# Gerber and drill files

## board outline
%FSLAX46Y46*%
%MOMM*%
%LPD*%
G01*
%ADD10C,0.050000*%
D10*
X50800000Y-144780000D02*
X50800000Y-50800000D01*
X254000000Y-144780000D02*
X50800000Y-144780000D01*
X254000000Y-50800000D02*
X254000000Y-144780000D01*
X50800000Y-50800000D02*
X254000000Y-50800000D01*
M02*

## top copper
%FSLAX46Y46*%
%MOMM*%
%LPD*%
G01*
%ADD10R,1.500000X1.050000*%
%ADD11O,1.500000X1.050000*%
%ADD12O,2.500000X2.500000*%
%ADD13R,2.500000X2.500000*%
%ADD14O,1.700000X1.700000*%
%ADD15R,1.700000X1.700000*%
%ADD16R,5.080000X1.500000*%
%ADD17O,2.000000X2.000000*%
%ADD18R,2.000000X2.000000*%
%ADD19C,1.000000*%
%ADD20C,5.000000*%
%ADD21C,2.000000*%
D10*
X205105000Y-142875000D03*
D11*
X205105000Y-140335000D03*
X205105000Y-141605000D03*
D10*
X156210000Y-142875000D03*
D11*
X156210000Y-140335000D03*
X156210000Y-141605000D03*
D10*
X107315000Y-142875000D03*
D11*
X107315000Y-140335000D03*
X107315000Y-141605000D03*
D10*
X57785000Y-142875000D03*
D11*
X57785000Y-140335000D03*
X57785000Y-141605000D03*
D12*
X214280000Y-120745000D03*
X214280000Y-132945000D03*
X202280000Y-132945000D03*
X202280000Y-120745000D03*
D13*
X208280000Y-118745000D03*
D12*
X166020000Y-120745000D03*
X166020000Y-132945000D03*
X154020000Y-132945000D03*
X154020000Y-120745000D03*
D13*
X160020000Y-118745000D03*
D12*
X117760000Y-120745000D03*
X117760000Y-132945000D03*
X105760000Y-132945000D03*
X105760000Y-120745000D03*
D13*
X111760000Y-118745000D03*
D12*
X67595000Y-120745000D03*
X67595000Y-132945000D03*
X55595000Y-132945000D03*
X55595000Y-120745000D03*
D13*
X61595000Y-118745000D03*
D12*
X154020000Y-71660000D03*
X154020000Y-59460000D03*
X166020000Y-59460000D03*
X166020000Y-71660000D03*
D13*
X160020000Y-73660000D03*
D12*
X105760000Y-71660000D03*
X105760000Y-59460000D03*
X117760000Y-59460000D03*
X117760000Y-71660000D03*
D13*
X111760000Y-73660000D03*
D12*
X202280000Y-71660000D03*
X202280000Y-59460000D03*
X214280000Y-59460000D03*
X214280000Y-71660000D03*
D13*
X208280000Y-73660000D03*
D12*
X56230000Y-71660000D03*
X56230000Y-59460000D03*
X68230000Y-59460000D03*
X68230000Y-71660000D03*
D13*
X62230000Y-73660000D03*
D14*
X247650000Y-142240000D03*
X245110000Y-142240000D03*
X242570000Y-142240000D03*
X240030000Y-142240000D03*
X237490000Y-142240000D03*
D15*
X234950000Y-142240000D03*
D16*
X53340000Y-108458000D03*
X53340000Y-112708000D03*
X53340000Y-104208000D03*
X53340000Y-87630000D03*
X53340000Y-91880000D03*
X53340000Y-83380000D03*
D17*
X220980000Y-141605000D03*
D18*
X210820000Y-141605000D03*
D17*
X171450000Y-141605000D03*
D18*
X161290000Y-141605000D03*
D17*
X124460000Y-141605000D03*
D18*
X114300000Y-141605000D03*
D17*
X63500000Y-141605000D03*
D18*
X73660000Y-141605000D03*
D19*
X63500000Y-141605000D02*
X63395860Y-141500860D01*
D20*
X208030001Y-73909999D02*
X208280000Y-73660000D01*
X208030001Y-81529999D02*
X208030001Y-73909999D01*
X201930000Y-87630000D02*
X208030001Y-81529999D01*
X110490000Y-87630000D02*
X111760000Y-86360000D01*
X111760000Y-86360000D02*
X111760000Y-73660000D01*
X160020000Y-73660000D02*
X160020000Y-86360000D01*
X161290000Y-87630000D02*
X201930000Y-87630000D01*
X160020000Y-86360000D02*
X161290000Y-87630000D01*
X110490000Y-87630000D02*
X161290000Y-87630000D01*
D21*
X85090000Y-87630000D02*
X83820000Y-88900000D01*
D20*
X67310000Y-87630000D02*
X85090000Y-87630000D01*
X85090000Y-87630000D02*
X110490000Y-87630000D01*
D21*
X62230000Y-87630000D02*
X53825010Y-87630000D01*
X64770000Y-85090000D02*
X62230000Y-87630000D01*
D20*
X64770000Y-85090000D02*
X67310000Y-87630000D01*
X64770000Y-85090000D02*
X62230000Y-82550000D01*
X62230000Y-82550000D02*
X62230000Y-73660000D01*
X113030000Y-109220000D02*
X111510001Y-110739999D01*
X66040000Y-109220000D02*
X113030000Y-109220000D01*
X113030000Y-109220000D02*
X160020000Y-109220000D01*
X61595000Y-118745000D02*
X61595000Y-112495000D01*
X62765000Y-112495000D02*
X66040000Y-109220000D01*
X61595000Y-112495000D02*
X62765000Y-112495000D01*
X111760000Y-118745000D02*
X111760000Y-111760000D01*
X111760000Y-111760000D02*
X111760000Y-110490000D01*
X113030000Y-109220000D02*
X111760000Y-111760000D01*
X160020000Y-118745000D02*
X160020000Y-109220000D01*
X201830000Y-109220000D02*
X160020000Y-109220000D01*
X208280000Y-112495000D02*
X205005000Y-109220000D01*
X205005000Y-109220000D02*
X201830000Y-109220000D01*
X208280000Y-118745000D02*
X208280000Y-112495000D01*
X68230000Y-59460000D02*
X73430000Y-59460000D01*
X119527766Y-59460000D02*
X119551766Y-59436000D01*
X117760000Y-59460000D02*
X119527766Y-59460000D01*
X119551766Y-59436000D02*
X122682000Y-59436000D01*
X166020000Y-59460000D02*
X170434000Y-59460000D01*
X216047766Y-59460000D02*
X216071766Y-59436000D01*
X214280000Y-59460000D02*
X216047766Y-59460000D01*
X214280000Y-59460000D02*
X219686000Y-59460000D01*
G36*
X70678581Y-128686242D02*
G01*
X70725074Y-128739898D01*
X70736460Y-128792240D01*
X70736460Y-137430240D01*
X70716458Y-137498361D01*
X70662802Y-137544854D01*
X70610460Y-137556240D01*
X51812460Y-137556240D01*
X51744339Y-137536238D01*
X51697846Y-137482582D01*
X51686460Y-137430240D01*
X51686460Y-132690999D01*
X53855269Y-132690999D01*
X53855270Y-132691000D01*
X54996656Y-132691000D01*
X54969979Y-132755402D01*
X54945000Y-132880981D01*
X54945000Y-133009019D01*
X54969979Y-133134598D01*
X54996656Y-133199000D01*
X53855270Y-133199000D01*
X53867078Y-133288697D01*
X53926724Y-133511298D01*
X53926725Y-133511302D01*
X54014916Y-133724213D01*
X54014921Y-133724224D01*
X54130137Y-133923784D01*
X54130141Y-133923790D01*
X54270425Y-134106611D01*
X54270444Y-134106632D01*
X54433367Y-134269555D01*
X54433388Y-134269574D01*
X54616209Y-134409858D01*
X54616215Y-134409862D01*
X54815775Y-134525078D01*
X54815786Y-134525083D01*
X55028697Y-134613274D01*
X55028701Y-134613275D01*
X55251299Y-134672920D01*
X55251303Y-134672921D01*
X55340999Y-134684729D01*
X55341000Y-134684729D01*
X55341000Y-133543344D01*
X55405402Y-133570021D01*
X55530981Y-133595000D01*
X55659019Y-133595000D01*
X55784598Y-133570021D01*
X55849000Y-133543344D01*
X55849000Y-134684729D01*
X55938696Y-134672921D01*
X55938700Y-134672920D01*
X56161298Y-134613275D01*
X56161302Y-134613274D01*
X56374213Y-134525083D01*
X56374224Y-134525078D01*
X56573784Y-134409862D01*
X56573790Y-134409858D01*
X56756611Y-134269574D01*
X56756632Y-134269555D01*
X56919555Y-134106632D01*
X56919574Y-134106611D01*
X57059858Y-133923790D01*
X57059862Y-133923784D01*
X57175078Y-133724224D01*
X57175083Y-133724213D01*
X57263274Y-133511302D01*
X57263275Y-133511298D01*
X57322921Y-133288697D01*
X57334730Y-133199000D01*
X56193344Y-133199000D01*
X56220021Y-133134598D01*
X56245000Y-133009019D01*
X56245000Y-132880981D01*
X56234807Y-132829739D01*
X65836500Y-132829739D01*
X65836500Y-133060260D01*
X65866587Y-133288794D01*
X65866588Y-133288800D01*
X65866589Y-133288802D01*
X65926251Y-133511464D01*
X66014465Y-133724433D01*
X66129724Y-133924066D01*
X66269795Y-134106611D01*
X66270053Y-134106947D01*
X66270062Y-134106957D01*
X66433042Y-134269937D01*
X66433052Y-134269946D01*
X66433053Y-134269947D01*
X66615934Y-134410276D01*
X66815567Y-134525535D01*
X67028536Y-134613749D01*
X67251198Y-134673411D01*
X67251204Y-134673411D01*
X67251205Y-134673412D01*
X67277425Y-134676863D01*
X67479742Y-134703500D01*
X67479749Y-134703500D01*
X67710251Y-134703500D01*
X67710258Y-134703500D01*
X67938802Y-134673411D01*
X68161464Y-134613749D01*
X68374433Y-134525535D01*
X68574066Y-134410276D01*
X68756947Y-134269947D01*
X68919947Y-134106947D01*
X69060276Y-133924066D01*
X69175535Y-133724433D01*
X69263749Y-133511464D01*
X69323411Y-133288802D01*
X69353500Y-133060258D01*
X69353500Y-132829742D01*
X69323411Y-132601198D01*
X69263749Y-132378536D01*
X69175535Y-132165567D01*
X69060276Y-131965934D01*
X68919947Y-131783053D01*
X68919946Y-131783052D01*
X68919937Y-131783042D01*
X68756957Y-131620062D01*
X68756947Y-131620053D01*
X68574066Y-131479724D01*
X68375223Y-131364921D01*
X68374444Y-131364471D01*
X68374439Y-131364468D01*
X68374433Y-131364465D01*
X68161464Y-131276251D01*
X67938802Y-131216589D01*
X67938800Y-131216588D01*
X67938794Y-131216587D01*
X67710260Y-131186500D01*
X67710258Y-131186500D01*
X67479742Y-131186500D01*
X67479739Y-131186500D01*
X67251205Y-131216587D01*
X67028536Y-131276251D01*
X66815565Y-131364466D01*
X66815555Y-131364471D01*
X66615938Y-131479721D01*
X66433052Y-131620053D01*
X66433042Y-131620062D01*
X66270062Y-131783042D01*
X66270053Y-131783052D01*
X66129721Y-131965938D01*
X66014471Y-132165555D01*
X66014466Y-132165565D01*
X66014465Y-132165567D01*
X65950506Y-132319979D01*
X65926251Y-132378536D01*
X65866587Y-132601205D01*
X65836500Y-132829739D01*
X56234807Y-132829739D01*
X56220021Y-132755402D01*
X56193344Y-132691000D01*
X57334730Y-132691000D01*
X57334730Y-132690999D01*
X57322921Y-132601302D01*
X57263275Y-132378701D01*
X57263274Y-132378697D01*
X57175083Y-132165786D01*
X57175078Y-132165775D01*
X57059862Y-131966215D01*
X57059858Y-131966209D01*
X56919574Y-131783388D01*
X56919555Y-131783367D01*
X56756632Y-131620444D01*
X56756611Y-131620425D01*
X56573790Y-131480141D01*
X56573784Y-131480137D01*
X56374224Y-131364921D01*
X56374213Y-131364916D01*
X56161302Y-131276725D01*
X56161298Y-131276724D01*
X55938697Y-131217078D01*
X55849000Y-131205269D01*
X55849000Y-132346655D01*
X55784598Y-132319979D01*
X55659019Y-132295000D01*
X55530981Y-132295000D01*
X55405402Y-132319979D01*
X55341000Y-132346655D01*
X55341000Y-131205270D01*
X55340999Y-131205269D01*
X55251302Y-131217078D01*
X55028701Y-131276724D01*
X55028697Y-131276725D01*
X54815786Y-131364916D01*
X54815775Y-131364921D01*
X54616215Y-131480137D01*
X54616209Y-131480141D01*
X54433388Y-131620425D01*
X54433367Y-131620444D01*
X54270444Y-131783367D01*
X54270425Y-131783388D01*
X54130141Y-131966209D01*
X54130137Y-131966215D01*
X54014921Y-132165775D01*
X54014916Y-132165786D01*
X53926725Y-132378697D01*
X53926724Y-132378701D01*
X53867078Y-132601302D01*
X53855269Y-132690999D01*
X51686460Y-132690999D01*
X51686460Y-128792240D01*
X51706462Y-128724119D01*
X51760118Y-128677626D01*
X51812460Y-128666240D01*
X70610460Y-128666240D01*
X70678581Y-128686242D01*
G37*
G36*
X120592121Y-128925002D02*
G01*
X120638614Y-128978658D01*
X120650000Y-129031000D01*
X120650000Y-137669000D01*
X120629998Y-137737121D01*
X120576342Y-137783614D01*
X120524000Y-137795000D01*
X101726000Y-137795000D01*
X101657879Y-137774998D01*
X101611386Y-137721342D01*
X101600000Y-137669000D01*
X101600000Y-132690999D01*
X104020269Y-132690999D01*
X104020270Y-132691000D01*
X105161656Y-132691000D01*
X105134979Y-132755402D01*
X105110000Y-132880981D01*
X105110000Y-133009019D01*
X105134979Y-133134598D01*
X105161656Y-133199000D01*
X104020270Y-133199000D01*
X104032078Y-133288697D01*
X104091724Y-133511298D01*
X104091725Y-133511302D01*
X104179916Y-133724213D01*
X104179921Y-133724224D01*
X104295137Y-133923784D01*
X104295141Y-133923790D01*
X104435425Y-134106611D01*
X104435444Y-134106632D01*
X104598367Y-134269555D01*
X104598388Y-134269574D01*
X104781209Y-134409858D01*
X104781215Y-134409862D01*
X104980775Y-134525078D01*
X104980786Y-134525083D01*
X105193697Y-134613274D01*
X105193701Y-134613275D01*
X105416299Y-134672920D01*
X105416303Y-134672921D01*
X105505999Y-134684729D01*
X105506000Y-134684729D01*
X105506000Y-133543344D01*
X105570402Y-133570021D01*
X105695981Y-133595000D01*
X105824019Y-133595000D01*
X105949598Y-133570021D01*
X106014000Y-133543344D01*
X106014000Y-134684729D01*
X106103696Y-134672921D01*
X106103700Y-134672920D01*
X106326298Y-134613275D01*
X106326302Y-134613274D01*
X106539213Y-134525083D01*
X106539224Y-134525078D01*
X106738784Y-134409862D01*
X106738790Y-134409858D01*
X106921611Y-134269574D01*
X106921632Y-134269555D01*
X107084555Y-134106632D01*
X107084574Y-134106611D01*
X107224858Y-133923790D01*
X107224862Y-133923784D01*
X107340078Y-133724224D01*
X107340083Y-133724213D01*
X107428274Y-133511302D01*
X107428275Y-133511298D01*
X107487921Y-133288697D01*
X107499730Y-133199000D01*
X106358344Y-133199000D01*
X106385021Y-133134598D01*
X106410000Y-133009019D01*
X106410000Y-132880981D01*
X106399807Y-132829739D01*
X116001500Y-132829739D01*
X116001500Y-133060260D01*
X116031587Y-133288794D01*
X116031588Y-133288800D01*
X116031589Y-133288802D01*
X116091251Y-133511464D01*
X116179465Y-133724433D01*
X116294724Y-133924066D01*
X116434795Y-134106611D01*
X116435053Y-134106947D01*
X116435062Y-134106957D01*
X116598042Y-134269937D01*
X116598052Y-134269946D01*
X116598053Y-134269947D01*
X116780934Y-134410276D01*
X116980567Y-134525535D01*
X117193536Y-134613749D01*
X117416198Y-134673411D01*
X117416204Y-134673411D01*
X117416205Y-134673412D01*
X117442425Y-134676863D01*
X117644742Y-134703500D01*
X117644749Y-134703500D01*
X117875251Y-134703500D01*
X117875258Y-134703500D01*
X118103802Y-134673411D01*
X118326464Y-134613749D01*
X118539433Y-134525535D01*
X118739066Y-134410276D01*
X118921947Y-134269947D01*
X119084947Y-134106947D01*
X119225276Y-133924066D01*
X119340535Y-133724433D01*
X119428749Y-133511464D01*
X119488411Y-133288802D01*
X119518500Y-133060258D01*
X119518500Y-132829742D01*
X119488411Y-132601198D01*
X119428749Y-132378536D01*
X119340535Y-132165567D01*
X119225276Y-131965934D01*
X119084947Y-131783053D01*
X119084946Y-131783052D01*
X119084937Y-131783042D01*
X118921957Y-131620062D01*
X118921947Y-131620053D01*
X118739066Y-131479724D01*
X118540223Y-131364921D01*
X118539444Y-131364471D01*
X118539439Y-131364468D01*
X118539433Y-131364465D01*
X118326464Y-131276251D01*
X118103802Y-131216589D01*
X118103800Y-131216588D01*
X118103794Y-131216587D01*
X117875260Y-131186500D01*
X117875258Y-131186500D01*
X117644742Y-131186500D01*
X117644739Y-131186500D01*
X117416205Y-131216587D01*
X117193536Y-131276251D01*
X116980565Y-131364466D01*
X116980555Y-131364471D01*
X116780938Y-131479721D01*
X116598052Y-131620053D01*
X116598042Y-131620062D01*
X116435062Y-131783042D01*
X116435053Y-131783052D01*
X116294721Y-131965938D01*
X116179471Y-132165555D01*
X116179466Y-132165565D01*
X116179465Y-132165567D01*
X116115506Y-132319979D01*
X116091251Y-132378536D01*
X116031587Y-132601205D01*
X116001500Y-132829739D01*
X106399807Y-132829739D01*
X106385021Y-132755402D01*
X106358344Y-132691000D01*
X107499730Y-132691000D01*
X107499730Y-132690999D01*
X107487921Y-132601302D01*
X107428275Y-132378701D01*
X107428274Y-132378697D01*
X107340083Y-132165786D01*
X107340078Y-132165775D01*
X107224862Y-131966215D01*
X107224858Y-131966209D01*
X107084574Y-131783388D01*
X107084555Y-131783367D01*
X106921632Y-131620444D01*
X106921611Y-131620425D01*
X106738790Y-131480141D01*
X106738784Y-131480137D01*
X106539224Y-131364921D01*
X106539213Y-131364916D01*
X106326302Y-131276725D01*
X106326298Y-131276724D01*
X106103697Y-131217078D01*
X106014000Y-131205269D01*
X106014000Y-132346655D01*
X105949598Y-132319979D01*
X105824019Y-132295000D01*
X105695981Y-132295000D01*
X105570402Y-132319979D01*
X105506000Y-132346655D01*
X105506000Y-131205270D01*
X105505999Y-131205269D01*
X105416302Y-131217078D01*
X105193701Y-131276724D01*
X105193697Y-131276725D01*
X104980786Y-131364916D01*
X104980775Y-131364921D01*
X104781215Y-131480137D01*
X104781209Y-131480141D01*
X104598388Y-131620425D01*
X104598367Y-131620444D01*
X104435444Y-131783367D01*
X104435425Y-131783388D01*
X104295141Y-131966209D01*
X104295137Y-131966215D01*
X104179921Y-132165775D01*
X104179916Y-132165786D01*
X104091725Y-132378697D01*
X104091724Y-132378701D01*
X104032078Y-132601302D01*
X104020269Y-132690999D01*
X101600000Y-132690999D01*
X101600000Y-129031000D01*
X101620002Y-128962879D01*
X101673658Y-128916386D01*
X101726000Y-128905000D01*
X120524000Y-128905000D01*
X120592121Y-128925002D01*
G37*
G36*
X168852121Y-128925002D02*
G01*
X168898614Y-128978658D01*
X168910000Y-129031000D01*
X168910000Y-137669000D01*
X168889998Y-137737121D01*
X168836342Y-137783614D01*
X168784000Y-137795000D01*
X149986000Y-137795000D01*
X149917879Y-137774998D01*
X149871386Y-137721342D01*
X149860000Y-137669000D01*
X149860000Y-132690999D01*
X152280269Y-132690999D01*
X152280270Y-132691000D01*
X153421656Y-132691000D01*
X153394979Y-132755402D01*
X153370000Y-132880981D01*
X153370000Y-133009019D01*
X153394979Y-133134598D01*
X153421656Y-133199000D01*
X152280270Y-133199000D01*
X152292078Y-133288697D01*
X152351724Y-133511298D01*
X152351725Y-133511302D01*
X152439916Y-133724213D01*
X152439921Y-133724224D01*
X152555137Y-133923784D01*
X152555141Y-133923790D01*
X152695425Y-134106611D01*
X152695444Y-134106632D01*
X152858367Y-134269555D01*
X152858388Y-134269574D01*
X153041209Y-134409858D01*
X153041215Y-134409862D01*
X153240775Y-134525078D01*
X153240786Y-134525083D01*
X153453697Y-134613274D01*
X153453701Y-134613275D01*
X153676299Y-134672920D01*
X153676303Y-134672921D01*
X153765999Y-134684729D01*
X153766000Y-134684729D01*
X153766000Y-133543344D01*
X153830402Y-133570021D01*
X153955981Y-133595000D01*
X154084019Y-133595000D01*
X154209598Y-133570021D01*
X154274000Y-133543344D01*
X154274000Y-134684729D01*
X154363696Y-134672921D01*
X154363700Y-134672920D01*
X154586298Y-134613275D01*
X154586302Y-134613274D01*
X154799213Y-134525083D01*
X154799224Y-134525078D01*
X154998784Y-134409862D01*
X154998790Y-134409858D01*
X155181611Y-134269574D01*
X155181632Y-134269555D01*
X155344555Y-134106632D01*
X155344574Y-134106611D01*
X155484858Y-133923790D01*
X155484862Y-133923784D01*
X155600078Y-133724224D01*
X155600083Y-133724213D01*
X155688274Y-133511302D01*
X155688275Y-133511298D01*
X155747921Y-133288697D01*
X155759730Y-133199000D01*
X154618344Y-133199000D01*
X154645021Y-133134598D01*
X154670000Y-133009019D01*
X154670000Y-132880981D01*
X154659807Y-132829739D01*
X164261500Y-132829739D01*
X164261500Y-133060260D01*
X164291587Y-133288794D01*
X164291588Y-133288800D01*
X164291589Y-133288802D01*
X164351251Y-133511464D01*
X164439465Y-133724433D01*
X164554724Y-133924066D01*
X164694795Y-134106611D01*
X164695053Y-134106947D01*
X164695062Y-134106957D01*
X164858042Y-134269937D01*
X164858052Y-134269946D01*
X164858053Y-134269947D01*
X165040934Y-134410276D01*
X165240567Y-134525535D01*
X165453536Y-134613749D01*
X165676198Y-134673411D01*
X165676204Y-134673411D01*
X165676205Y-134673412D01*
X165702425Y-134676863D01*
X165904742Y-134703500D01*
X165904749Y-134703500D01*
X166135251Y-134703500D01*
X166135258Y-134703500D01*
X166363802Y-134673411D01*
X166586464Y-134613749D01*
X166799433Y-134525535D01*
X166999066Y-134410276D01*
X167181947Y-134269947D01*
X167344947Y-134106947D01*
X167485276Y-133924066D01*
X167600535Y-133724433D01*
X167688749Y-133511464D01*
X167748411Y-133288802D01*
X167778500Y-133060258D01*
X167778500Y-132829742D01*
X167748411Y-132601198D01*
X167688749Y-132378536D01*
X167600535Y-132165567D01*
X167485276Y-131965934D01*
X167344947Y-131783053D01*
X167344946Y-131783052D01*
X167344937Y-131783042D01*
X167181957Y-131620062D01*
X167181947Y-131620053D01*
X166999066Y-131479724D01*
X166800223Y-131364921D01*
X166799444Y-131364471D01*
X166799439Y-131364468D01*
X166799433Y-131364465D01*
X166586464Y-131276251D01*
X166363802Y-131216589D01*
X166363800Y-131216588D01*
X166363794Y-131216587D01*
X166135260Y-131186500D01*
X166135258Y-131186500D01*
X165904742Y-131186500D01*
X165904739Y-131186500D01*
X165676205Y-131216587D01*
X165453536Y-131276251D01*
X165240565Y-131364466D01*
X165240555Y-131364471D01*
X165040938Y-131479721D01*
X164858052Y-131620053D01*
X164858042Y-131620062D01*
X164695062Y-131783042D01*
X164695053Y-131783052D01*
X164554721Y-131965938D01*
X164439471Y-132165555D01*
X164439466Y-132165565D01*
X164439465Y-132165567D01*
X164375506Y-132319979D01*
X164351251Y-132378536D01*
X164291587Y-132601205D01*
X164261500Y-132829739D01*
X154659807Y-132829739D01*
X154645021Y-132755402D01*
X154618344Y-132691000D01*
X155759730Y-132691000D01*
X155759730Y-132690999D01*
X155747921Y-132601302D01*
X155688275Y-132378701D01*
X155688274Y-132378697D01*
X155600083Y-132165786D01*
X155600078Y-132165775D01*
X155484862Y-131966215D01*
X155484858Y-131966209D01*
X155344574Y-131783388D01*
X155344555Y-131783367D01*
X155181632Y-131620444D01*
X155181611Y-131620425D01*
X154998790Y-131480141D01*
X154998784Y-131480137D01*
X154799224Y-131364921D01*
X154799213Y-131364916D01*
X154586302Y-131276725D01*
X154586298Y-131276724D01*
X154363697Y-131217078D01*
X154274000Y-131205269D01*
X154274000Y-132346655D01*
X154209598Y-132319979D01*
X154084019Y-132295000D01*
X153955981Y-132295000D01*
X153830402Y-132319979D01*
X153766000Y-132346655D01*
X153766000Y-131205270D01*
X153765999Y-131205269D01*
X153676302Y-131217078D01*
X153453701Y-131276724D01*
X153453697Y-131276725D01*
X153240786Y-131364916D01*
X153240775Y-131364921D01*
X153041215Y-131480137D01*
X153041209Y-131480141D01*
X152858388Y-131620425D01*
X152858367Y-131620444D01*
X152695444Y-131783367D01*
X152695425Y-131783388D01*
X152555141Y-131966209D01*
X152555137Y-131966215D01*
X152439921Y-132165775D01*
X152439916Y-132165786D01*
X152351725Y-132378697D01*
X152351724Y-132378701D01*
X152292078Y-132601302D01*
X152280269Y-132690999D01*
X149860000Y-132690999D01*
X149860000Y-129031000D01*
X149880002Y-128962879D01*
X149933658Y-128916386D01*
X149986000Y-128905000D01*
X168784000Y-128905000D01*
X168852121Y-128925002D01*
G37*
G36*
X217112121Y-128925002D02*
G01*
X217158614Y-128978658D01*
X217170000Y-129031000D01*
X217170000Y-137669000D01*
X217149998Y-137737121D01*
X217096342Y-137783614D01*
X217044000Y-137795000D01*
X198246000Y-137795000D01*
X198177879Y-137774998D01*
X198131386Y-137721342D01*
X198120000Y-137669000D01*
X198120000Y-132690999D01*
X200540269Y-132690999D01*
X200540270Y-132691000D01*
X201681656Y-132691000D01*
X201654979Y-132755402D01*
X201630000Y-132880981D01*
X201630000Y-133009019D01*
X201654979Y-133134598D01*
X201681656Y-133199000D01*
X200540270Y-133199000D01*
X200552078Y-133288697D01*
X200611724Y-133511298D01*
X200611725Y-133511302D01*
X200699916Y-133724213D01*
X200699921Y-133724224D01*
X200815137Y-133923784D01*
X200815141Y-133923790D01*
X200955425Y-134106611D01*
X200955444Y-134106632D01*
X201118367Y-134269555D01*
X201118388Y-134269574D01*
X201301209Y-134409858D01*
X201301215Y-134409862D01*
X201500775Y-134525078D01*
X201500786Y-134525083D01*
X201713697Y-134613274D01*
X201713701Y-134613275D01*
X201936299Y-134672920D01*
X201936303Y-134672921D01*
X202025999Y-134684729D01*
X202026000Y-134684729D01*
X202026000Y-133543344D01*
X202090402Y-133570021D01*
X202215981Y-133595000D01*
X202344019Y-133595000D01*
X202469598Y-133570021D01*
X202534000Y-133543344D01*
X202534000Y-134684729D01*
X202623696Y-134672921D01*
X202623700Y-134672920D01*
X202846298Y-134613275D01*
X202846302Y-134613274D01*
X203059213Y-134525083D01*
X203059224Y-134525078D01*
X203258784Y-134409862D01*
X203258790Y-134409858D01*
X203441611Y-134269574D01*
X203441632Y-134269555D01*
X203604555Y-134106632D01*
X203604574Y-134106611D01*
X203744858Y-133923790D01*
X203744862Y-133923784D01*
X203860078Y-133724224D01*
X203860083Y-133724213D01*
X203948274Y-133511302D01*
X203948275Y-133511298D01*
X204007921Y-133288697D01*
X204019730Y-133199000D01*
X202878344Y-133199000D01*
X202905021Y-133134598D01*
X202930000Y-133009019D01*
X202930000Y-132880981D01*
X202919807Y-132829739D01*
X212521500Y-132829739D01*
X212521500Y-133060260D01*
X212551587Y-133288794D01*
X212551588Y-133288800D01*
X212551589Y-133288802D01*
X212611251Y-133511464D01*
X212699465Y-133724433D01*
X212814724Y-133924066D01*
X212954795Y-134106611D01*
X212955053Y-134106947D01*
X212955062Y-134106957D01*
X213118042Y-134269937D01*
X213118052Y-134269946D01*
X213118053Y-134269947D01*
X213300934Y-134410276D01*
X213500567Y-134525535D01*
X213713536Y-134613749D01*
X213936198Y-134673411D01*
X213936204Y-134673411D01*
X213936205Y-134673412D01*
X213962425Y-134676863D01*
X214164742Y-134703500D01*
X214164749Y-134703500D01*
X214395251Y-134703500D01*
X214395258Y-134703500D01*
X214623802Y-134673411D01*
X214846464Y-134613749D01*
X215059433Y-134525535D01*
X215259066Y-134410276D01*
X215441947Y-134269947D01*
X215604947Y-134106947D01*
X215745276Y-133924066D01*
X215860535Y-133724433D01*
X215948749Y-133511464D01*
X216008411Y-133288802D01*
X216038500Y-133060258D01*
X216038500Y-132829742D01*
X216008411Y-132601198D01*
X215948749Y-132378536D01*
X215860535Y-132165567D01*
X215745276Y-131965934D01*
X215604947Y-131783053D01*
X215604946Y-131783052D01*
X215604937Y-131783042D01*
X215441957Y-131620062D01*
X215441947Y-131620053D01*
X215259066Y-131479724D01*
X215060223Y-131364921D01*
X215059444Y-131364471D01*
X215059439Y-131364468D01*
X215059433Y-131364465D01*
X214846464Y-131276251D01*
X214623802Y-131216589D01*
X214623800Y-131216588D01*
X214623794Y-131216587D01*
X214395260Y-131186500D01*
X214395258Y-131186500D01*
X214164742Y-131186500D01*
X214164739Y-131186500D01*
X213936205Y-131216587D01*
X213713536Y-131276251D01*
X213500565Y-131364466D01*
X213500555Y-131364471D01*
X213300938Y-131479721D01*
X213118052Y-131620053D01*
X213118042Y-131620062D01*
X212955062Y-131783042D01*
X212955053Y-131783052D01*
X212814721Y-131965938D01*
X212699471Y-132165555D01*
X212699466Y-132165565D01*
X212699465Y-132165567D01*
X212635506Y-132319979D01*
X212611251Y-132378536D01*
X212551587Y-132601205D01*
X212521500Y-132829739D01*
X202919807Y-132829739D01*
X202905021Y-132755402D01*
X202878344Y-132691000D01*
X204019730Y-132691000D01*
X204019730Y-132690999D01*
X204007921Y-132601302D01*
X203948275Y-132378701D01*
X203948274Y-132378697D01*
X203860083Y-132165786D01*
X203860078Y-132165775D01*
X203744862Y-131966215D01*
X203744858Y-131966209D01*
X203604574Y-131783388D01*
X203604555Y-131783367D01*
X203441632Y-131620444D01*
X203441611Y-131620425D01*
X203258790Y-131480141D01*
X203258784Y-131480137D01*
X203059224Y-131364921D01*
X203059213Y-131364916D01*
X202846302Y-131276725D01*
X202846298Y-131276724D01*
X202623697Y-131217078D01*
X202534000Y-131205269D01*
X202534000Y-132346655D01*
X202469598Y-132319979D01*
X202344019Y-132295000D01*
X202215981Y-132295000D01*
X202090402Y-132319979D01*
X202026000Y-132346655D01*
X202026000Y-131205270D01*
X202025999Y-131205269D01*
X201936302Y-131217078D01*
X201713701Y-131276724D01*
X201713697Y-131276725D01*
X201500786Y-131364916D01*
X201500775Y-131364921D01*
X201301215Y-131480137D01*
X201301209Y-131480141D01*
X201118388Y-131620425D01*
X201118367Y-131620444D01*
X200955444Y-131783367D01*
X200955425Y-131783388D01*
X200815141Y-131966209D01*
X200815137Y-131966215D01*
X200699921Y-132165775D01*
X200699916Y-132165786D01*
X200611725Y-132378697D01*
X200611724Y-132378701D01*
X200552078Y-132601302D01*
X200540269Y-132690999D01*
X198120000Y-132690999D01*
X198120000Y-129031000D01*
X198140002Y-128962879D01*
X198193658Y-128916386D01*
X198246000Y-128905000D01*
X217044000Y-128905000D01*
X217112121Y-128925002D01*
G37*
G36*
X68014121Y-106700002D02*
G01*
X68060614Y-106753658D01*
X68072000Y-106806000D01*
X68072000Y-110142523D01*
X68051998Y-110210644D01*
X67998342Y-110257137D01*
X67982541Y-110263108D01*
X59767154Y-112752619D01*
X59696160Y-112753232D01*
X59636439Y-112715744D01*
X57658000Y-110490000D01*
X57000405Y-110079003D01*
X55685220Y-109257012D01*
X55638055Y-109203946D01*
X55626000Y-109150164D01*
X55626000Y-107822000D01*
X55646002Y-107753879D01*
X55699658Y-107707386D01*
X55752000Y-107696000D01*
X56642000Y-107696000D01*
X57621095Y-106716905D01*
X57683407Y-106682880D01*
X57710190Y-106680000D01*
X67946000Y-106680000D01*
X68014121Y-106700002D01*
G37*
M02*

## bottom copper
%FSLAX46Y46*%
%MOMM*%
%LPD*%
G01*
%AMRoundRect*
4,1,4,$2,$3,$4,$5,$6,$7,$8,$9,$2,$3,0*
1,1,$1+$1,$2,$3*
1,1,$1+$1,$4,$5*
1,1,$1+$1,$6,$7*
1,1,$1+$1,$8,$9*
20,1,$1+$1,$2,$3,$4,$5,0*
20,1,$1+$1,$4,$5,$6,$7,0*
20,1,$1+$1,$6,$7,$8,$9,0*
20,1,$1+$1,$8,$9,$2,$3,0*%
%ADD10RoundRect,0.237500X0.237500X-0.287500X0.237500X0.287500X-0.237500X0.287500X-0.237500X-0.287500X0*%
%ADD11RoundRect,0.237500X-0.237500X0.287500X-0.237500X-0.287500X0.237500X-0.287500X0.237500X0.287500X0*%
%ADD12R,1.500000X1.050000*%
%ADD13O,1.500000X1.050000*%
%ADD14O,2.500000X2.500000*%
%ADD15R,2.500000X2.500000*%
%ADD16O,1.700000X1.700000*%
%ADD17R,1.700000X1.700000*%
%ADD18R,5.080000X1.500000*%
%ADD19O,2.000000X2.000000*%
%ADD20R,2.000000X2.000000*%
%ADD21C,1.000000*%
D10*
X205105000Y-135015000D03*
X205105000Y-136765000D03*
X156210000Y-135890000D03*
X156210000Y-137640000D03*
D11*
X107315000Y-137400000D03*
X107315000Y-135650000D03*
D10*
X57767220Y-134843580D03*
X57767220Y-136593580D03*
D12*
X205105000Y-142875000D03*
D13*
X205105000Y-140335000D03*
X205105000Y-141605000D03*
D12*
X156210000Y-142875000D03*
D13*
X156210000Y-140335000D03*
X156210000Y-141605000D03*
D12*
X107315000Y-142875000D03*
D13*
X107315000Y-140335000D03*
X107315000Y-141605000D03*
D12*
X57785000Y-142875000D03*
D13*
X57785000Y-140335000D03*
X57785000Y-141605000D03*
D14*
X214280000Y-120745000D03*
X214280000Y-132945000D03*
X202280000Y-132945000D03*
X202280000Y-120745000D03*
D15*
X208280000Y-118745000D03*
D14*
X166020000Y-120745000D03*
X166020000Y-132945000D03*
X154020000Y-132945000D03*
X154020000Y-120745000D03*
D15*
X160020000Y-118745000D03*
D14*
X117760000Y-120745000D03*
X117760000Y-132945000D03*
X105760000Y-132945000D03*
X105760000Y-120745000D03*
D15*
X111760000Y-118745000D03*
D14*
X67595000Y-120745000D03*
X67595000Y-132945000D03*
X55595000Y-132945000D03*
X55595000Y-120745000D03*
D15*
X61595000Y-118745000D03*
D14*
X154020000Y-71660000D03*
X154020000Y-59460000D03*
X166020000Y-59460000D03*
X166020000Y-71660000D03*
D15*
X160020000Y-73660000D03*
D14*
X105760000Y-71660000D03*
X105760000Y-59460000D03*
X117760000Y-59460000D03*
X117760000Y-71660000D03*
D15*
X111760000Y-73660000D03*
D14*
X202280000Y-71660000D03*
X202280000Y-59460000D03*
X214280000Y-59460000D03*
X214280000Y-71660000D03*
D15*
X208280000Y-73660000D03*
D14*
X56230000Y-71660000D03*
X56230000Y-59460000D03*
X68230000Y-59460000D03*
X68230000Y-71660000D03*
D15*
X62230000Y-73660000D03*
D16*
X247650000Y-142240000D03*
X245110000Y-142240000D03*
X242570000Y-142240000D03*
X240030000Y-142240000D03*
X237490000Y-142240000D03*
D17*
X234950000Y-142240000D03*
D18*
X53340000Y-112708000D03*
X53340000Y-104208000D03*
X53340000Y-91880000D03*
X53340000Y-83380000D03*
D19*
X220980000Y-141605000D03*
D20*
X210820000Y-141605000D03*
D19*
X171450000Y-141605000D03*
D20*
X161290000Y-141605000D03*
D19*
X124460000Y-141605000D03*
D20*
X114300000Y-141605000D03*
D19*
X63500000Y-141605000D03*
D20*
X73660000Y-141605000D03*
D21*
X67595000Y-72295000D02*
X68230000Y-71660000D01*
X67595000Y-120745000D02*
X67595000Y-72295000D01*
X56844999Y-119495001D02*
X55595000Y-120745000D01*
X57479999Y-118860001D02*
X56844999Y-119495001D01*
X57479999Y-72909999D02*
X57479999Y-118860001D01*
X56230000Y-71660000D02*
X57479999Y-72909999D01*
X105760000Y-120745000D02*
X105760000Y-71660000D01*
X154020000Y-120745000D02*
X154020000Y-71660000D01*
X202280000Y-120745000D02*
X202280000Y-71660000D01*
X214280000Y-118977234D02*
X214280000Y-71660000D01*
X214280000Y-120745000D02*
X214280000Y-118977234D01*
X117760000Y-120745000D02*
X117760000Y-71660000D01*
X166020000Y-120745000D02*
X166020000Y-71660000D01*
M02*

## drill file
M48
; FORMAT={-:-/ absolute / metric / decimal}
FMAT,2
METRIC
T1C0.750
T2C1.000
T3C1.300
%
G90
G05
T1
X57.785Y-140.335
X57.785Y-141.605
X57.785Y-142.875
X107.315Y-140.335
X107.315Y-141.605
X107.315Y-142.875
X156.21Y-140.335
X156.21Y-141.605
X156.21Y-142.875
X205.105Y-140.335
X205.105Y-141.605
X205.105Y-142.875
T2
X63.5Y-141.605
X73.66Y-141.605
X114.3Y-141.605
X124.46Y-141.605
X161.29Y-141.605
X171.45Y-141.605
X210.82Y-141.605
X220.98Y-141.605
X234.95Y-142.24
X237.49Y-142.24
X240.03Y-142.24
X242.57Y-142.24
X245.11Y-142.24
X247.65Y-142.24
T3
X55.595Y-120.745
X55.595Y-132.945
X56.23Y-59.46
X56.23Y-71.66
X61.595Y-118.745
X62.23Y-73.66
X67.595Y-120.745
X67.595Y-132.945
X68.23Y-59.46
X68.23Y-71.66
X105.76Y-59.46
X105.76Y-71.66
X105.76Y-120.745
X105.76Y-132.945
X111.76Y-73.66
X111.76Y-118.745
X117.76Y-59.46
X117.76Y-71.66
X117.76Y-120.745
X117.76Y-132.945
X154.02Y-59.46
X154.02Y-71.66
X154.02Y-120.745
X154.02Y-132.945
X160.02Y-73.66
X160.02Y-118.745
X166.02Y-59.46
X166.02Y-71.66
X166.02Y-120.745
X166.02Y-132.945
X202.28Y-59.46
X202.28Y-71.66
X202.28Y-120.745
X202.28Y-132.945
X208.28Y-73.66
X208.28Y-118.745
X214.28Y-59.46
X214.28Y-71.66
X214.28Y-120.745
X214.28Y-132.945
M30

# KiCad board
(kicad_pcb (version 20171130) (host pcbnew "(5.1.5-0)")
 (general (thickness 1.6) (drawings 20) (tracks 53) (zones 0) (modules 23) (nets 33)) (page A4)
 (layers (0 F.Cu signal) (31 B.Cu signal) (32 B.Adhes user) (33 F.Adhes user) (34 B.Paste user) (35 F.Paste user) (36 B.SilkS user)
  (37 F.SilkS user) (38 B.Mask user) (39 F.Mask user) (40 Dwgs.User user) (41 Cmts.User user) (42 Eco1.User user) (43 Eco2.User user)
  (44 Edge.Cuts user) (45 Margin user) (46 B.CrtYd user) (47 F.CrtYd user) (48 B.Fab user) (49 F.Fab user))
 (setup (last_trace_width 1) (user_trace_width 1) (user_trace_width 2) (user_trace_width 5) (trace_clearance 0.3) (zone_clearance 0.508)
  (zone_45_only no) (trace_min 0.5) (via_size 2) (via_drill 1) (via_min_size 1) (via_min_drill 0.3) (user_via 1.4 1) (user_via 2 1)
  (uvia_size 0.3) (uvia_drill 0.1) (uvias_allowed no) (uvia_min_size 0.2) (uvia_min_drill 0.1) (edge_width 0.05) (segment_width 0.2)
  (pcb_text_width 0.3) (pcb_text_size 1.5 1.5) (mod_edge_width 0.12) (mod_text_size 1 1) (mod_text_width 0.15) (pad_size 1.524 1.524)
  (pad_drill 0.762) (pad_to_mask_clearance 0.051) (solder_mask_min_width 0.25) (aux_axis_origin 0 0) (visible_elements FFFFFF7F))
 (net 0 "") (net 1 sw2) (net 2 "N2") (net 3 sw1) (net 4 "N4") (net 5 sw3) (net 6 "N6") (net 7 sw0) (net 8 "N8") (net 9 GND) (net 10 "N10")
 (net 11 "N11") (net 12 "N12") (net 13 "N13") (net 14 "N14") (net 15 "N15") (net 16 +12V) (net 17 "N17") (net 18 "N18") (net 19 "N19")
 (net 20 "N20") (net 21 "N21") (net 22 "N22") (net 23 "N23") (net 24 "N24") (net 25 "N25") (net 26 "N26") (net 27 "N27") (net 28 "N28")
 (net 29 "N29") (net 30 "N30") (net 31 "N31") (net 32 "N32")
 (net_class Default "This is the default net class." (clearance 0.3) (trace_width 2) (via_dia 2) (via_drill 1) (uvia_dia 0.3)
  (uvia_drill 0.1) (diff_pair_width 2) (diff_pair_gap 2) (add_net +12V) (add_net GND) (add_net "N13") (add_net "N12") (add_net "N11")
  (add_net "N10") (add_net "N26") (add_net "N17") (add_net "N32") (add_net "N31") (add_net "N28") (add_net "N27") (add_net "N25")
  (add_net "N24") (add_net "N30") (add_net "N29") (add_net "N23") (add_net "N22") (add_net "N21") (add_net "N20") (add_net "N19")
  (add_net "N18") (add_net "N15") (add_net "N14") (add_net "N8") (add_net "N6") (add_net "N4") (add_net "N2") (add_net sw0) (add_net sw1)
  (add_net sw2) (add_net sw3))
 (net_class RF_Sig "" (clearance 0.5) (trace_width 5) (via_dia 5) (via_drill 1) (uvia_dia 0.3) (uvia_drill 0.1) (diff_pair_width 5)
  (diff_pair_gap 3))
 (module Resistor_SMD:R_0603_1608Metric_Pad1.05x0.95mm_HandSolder (layer B.Cu) (at 205.105 135.89 90)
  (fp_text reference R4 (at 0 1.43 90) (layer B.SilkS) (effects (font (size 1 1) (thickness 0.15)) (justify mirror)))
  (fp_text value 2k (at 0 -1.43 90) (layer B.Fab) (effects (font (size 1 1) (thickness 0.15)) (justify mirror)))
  (pad 2 smd roundrect (at 0.875 0 90) (size 1.05 0.95) (layers B.Cu B.Paste B.Mask) (roundrect_rratio 0.25) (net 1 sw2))
  (pad 1 smd roundrect (at -0.875 0 90) (size 1.05 0.95) (layers B.Cu B.Paste B.Mask) (roundrect_rratio 0.25) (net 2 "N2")))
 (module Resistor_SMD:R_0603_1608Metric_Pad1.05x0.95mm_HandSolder (layer B.Cu) (at 156.21 136.765 90)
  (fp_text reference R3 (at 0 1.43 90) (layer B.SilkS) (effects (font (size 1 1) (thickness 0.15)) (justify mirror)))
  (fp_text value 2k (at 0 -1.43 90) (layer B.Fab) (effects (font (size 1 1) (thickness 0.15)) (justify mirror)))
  (pad 2 smd roundrect (at 0.875 0 90) (size 1.05 0.95) (layers B.Cu B.Paste B.Mask) (roundrect_rratio 0.25) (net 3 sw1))
  (pad 1 smd roundrect (at -0.875 0 90) (size 1.05 0.95) (layers B.Cu B.Paste B.Mask) (roundrect_rratio 0.25) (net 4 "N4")))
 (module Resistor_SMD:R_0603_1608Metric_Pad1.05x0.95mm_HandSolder (layer B.Cu) (at 107.315 136.525 270)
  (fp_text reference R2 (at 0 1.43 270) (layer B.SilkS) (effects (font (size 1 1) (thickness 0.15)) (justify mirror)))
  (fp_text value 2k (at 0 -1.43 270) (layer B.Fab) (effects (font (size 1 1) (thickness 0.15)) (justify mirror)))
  (pad 2 smd roundrect (at 0.875 0 270) (size 1.05 0.95) (layers B.Cu B.Paste B.Mask) (roundrect_rratio 0.25) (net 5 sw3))
  (pad 1 smd roundrect (at -0.875 0 270) (size 1.05 0.95) (layers B.Cu B.Paste B.Mask) (roundrect_rratio 0.25) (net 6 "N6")))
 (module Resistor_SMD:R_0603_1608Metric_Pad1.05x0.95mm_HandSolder (layer B.Cu) (at 57.76722 135.71858 90)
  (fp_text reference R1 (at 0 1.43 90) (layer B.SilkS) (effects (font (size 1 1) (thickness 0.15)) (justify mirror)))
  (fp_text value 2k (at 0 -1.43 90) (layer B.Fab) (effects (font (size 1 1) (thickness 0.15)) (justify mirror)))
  (pad 2 smd roundrect (at 0.875 0 90) (size 1.05 0.95) (layers B.Cu B.Paste B.Mask) (roundrect_rratio 0.25) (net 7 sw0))
  (pad 1 smd roundrect (at -0.875 0 90) (size 1.05 0.95) (layers B.Cu B.Paste B.Mask) (roundrect_rratio 0.25) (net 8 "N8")))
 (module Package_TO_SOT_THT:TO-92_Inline (layer F.Cu) (at 205.105 142.875 90)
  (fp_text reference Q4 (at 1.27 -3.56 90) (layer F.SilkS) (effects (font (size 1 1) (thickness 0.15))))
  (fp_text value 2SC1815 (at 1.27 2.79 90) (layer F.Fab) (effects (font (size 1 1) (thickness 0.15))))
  (pad 1 thru_hole rect (at 0 0 90) (size 1.05 1.5) (drill 0.75) (layers *.Cu *.Mask) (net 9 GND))
  (pad 3 thru_hole oval (at 2.54 0 90) (size 1.05 1.5) (drill 0.75) (layers *.Cu *.Mask) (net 2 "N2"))
  (pad 2 thru_hole oval (at 1.27 0 90) (size 1.05 1.5) (drill 0.75) (layers *.Cu *.Mask) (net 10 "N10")))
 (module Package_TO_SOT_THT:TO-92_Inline (layer F.Cu) (at 156.21 142.875 90)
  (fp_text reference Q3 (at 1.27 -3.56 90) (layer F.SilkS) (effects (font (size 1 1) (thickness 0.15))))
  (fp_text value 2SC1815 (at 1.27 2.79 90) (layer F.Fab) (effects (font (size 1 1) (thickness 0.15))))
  (pad 1 thru_hole rect (at 0 0 90) (size 1.05 1.5) (drill 0.75) (layers *.Cu *.Mask) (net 9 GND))
  (pad 3 thru_hole oval (at 2.54 0 90) (size 1.05 1.5) (drill 0.75) (layers *.Cu *.Mask) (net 4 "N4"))
  (pad 2 thru_hole oval (at 1.27 0 90) (size 1.05 1.5) (drill 0.75) (layers *.Cu *.Mask) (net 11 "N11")))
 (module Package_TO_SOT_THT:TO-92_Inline (layer F.Cu) (at 107.315 142.875 90)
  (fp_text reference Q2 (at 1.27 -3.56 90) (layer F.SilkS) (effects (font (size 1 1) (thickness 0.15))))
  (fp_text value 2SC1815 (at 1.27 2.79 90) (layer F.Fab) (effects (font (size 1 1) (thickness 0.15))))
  (pad 1 thru_hole rect (at 0 0 90) (size 1.05 1.5) (drill 0.75) (layers *.Cu *.Mask) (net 9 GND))
  (pad 3 thru_hole oval (at 2.54 0 90) (size 1.05 1.5) (drill 0.75) (layers *.Cu *.Mask) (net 6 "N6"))
  (pad 2 thru_hole oval (at 1.27 0 90) (size 1.05 1.5) (drill 0.75) (layers *.Cu *.Mask) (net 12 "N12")))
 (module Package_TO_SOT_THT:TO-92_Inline (layer F.Cu) (at 57.785 142.875 90)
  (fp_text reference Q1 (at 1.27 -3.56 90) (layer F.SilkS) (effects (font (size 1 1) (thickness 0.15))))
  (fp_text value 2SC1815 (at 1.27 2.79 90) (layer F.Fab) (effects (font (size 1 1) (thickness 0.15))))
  (pad 1 thru_hole rect (at 0 0 90) (size 1.05 1.5) (drill 0.75) (layers *.Cu *.Mask) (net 9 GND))
  (pad 3 thru_hole oval (at 2.54 0 90) (size 1.05 1.5) (drill 0.75) (layers *.Cu *.Mask) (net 8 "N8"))
  (pad 2 thru_hole oval (at 1.27 0 90) (size 1.05 1.5) (drill 0.75) (layers *.Cu *.Mask) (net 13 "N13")))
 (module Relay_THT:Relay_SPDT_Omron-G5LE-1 (layer F.Cu) (at 208.28 118.745)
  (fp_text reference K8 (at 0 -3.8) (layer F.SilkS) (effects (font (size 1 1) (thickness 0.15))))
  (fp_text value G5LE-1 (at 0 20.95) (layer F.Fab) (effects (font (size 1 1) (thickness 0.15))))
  (pad 5 thru_hole oval (at 6 2) (size 2.5 2.5) (drill 1.3) (layers *.Cu *.Mask) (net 12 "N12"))
  (pad 4 thru_hole oval (at 6 14.2) (size 2.5 2.5) (drill 1.3) (layers *.Cu *.Mask) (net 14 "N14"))
  (pad 3 thru_hole oval (at -6 14.2) (size 2.5 2.5) (drill 1.3) (layers *.Cu *.Mask) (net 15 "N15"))
  (pad 2 thru_hole oval (at -6 2) (size 2.5 2.5) (drill 1.3) (layers *.Cu *.Mask) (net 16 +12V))
  (pad 1 thru_hole rect (at 0 0) (size 2.5 2.5) (drill 1.3) (layers *.Cu *.Mask) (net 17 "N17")))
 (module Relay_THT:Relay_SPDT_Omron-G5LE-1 (layer F.Cu) (at 160.02 118.745)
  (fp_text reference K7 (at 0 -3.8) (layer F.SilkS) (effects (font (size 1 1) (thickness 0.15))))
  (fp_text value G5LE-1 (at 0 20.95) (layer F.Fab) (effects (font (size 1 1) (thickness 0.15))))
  (pad 5 thru_hole oval (at 6 2) (size 2.5 2.5) (drill 1.3) (layers *.Cu *.Mask) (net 10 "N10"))
  (pad 4 thru_hole oval (at 6 14.2) (size 2.5 2.5) (drill 1.3) (layers *.Cu *.Mask) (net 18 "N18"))
  (pad 3 thru_hole oval (at -6 14.2) (size 2.5 2.5) (drill 1.3) (layers *.Cu *.Mask) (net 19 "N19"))
  (pad 2 thru_hole oval (at -6 2) (size 2.5 2.5) (drill 1.3) (layers *.Cu *.Mask) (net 16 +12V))
  (pad 1 thru_hole rect (at 0 0) (size 2.5 2.5) (drill 1.3) (layers *.Cu *.Mask) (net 17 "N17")))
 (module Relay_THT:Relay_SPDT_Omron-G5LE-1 (layer F.Cu) (at 111.76 118.745)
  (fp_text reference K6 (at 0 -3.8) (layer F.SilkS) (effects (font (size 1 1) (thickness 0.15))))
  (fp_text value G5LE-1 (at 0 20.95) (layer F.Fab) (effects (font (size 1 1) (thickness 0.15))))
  (pad 5 thru_hole oval (at 6 2) (size 2.5 2.5) (drill 1.3) (layers *.Cu *.Mask) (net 11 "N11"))
  (pad 4 thru_hole oval (at 6 14.2) (size 2.5 2.5) (drill 1.3) (layers *.Cu *.Mask) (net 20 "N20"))
  (pad 3 thru_hole oval (at -6 14.2) (size 2.5 2.5) (drill 1.3) (layers *.Cu *.Mask) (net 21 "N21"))
  (pad 2 thru_hole oval (at -6 2) (size 2.5 2.5) (drill 1.3) (layers *.Cu *.Mask) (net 16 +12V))
  (pad 1 thru_hole rect (at 0 0) (size 2.5 2.5) (drill 1.3) (layers *.Cu *.Mask) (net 17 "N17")))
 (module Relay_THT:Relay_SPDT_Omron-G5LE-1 (layer F.Cu) (at 61.595 118.745)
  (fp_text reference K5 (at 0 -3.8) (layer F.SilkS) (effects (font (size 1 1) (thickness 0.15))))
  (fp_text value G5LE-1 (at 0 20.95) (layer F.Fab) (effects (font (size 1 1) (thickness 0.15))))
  (pad 5 thru_hole oval (at 6 2) (size 2.5 2.5) (drill 1.3) (layers *.Cu *.Mask) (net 13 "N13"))
  (pad 4 thru_hole oval (at 6 14.2) (size 2.5 2.5) (drill 1.3) (layers *.Cu *.Mask) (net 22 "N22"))
  (pad 3 thru_hole oval (at -6 14.2) (size 2.5 2.5) (drill 1.3) (layers *.Cu *.Mask) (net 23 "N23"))
  (pad 2 thru_hole oval (at -6 2) (size 2.5 2.5) (drill 1.3) (layers *.Cu *.Mask) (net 16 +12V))
  (pad 1 thru_hole rect (at 0 0) (size 2.5 2.5) (drill 1.3) (layers *.Cu *.Mask) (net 17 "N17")))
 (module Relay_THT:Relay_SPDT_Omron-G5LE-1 (layer F.Cu) (at 160.02 73.66 180)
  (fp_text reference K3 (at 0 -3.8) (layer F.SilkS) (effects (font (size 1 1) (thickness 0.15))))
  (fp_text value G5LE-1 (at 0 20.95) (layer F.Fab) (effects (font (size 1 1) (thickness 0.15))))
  (pad 5 thru_hole oval (at 6 2 180) (size 2.5 2.5) (drill 1.3) (layers *.Cu *.Mask) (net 16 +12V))
  (pad 4 thru_hole oval (at 6 14.2 180) (size 2.5 2.5) (drill 1.3) (layers *.Cu *.Mask) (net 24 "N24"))
  (pad 3 thru_hole oval (at -6 14.2 180) (size 2.5 2.5) (drill 1.3) (layers *.Cu *.Mask) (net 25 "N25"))
  (pad 2 thru_hole oval (at -6 2 180) (size 2.5 2.5) (drill 1.3) (layers *.Cu *.Mask) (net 10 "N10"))
  (pad 1 thru_hole rect (at 0 0 180) (size 2.5 2.5) (drill 1.3) (layers *.Cu *.Mask) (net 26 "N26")))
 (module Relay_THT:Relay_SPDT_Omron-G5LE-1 (layer F.Cu) (at 111.76 73.66 180)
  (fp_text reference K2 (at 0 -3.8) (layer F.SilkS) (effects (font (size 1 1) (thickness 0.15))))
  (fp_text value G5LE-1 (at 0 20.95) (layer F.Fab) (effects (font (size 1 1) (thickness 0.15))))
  (pad 5 thru_hole oval (at 6 2 180) (size 2.5 2.5) (drill 1.3) (layers *.Cu *.Mask) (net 16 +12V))
  (pad 4 thru_hole oval (at 6 14.2 180) (size 2.5 2.5) (drill 1.3) (layers *.Cu *.Mask) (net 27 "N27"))
  (pad 3 thru_hole oval (at -6 14.2 180) (size 2.5 2.5) (drill 1.3) (layers *.Cu *.Mask) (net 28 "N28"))
  (pad 2 thru_hole oval (at -6 2 180) (size 2.5 2.5) (drill 1.3) (layers *.Cu *.Mask) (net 11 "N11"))
  (pad 1 thru_hole rect (at 0 0 180) (size 2.5 2.5) (drill 1.3) (layers *.Cu *.Mask) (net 26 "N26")))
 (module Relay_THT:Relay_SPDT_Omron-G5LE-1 (layer F.Cu) (at 208.28 73.66 180)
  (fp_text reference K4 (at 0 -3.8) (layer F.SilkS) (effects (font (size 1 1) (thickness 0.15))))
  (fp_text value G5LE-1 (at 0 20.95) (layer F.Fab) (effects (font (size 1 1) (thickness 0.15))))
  (pad 5 thru_hole oval (at 6 2 180) (size 2.5 2.5) (drill 1.3) (layers *.Cu *.Mask) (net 16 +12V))
  (pad 4 thru_hole oval (at 6 14.2 180) (size 2.5 2.5) (drill 1.3) (layers *.Cu *.Mask) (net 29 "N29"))
  (pad 3 thru_hole oval (at -6 14.2 180) (size 2.5 2.5) (drill 1.3) (layers *.Cu *.Mask) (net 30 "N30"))
  (pad 2 thru_hole oval (at -6 2 180) (size 2.5 2.5) (drill 1.3) (layers *.Cu *.Mask) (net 12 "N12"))
  (pad 1 thru_hole rect (at 0 0 180) (size 2.5 2.5) (drill 1.3) (layers *.Cu *.Mask) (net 26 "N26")))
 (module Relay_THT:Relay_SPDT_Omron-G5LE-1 (layer F.Cu) (at 62.23 73.66 180)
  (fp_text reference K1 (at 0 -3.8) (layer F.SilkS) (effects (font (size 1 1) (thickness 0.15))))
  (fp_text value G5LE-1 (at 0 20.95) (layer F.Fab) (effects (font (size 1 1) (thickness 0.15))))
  (pad 5 thru_hole oval (at 6 2 180) (size 2.5 2.5) (drill 1.3) (layers *.Cu *.Mask) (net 16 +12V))
  (pad 4 thru_hole oval (at 6 14.2 180) (size 2.5 2.5) (drill 1.3) (layers *.Cu *.Mask) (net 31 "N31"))
  (pad 3 thru_hole oval (at -6 14.2 180) (size 2.5 2.5) (drill 1.3) (layers *.Cu *.Mask) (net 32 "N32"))
  (pad 2 thru_hole oval (at -6 2 180) (size 2.5 2.5) (drill 1.3) (layers *.Cu *.Mask) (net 13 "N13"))
  (pad 1 thru_hole rect (at 0 0 180) (size 2.5 2.5) (drill 1.3) (layers *.Cu *.Mask) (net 26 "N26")))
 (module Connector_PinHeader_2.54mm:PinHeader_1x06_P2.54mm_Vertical (layer F.Cu) (at 234.95 142.24 90)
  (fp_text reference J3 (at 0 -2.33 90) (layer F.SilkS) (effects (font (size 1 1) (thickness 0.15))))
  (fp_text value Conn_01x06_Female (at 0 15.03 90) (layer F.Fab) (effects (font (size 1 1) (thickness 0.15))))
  (pad 6 thru_hole oval (at 0 12.7 90) (size 1.7 1.7) (drill 1) (layers *.Cu *.Mask) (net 9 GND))
  (pad 5 thru_hole oval (at 0 10.16 90) (size 1.7 1.7) (drill 1) (layers *.Cu *.Mask) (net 5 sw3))
  (pad 4 thru_hole oval (at 0 7.62 90) (size 1.7 1.7) (drill 1) (layers *.Cu *.Mask) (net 1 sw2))
  (pad 3 thru_hole oval (at 0 5.08 90) (size 1.7 1.7) (drill 1) (layers *.Cu *.Mask) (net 3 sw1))
  (pad 2 thru_hole oval (at 0 2.54 90) (size 1.7 1.7) (drill 1) (layers *.Cu *.Mask) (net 7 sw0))
  (pad 1 thru_hole rect (at 0 0 90) (size 1.7 1.7) (drill 1) (layers *.Cu *.Mask) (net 16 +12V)))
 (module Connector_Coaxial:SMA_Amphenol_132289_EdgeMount (layer F.Cu) (at 53.34 108.458 180)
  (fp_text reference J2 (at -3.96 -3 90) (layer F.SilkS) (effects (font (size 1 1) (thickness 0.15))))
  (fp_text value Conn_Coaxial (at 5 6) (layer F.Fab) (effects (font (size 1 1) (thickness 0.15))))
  (pad 1 smd rect (at 0 0 270) (size 1.5 5.08) (layers F.Cu F.Paste F.Mask) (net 17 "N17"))
  (pad 2 smd rect (at 0 -4.25 270) (size 1.5 5.08) (layers F.Cu F.Paste F.Mask) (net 9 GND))
  (pad 2 smd rect (at 0 4.25 270) (size 1.5 5.08) (layers F.Cu F.Paste F.Mask) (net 9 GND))
  (pad 2 smd rect (at 0 -4.25 270) (size 1.5 5.08) (layers B.Cu B.Paste B.Mask) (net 9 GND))
  (pad 2 smd rect (at 0 4.25 270) (size 1.5 5.08) (layers B.Cu B.Paste B.Mask) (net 9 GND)))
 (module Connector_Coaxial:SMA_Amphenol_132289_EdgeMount (layer F.Cu) (at 53.34 87.63 180)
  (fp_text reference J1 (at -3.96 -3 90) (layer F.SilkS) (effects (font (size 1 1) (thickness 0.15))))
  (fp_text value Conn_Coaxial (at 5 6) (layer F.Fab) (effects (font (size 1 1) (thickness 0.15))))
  (pad 1 smd rect (at 0 0 270) (size 1.5 5.08) (layers F.Cu F.Paste F.Mask) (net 26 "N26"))
  (pad 2 smd rect (at 0 -4.25 270) (size 1.5 5.08) (layers F.Cu F.Paste F.Mask) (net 9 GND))
  (pad 2 smd rect (at 0 4.25 270) (size 1.5 5.08) (layers F.Cu F.Paste F.Mask) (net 9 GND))
  (pad 2 smd rect (at 0 -4.25 270) (size 1.5 5.08) (layers B.Cu B.Paste B.Mask) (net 9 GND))
  (pad 2 smd rect (at 0 4.25 270) (size 1.5 5.08) (layers B.Cu B.Paste B.Mask) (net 9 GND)))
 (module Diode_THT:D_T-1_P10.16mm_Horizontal (layer F.Cu) (at 210.82 141.605)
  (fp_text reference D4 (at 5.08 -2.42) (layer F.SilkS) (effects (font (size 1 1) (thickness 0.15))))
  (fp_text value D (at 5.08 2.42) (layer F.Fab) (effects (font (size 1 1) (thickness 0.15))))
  (pad 2 thru_hole oval (at 10.16 0) (size 2 2) (drill 1) (layers *.Cu *.Mask) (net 10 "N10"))
  (pad 1 thru_hole rect (at 0 0) (size 2 2) (drill 1) (layers *.Cu *.Mask) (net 16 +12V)))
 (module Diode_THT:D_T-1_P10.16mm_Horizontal (layer F.Cu) (at 161.29 141.605)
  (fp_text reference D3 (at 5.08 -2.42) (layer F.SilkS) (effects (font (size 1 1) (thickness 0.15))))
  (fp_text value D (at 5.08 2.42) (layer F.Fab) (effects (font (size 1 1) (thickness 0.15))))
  (pad 2 thru_hole oval (at 10.16 0) (size 2 2) (drill 1) (layers *.Cu *.Mask) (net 11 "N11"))
  (pad 1 thru_hole rect (at 0 0) (size 2 2) (drill 1) (layers *.Cu *.Mask) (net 16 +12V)))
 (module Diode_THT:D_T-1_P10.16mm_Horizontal (layer F.Cu) (at 114.3 141.605)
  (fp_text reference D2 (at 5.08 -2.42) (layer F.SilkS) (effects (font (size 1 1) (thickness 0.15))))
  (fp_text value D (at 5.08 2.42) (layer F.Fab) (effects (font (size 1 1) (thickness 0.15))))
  (pad 2 thru_hole oval (at 10.16 0) (size 2 2) (drill 1) (layers *.Cu *.Mask) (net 12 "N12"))
  (pad 1 thru_hole rect (at 0 0) (size 2 2) (drill 1) (layers *.Cu *.Mask) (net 16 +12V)))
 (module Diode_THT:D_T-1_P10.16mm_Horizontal (layer F.Cu) (at 73.66 141.605 180)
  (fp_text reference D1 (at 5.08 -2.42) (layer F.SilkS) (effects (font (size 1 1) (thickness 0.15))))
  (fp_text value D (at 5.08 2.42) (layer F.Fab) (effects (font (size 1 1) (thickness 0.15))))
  (pad 2 thru_hole oval (at 10.16 0 180) (size 2 2) (drill 1) (layers *.Cu *.Mask) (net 13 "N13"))
  (pad 1 thru_hole rect (at 0 0 180) (size 2 2) (drill 1) (layers *.Cu *.Mask) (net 16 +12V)))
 (gr_line (start 50.8 144.78) (end 50.8 50.8) (layer Edge.Cuts) (width 0.05))
 (gr_line (start 254 144.78) (end 50.8 144.78) (layer Edge.Cuts) (width 0.05))
 (gr_line (start 254 50.8) (end 254 144.78) (layer Edge.Cuts) (width 0.05))
 (gr_line (start 50.8 50.8) (end 254 50.8) (layer Edge.Cuts) (width 0.05))
 (segment (start 63.5 141.605) (end 63.39586 141.50086) (width 1) (layer F.Cu) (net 13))
 (segment (start 67.595 72.295) (end 68.23 71.66) (width 1) (layer B.Cu) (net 13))
 (segment (start 67.595 120.745) (end 67.595 72.295) (width 1) (layer B.Cu) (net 13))
 (segment (start 56.844999 119.495001) (end 55.595 120.745) (width 1) (layer B.Cu) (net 16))
 (segment (start 57.479999 118.860001) (end 56.844999 119.495001) (width 1) (layer B.Cu) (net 16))
 (segment (start 57.479999 72.909999) (end 57.479999 118.860001) (width 1) (layer B.Cu) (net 16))
 (segment (start 56.23 71.66) (end 57.479999 72.909999) (width 1) (layer B.Cu) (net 16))
 (segment (start 105.76 120.745) (end 105.76 71.66) (width 1) (layer B.Cu) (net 16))
 (segment (start 154.02 120.745) (end 154.02 71.66) (width 1) (layer B.Cu) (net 16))
 (segment (start 202.28 120.745) (end 202.28 71.66) (width 1) (layer B.Cu) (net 16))
 (segment (start 214.28 118.977234) (end 214.28 71.66) (width 1) (layer B.Cu) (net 12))
 (segment (start 214.28 120.745) (end 214.28 118.977234) (width 1) (layer B.Cu) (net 12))
 (segment (start 117.76 120.745) (end 117.76 71.66) (width 1) (layer B.Cu) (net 11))
 (segment (start 166.02 120.745) (end 166.02 71.66) (width 1) (layer B.Cu) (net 10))
 (segment (start 208.030001 73.909999) (end 208.28 73.66) (width 5) (layer F.Cu) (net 26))
 (segment (start 208.030001 81.529999) (end 208.030001 73.909999) (width 5) (layer F.Cu) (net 26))
 (segment (start 201.93 87.63) (end 208.030001 81.529999) (width 5) (layer F.Cu) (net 26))
 (segment (start 110.49 87.63) (end 111.76 86.36) (width 5) (layer F.Cu) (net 26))
 (segment (start 111.76 86.36) (end 111.76 73.66) (width 5) (layer F.Cu) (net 26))
 (segment (start 160.02 73.66) (end 160.02 86.36) (width 5) (layer F.Cu) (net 26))
 (segment (start 161.29 87.63) (end 201.93 87.63) (width 5) (layer F.Cu) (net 26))
 (segment (start 160.02 86.36) (end 161.29 87.63) (width 5) (layer F.Cu) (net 26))
 (segment (start 110.49 87.63) (end 161.29 87.63) (width 5) (layer F.Cu) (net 26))
 (segment (start 85.09 87.63) (end 83.82 88.9) (width 2) (layer F.Cu) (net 26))
 (segment (start 67.31 87.63) (end 85.09 87.63) (width 5) (layer F.Cu) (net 26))
 (segment (start 85.09 87.63) (end 110.49 87.63) (width 5) (layer F.Cu) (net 26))
 (segment (start 62.23 87.63) (end 53.82501 87.63) (width 2) (layer F.Cu) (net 26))
 (segment (start 64.77 85.09) (end 62.23 87.63) (width 2) (layer F.Cu) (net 26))
 (segment (start 64.77 85.09) (end 67.31 87.63) (width 5) (layer F.Cu) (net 26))
 (segment (start 64.77 85.09) (end 62.23 82.55) (width 5) (layer F.Cu) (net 26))
 (segment (start 62.23 82.55) (end 62.23 73.66) (width 5) (layer F.Cu) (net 26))
 (segment (start 113.03 109.22) (end 111.510001 110.739999) (width 5) (layer F.Cu) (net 17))
 (segment (start 66.04 109.22) (end 113.03 109.22) (width 5) (layer F.Cu) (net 17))
 (segment (start 113.03 109.22) (end 160.02 109.22) (width 5) (layer F.Cu) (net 17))
 (segment (start 61.595 118.745) (end 61.595 112.495) (width 5) (layer F.Cu) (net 17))
 (segment (start 62.765 112.495) (end 66.04 109.22) (width 5) (layer F.Cu) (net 17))
 (segment (start 61.595 112.495) (end 62.765 112.495) (width 5) (layer F.Cu) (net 17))
 (segment (start 111.76 118.745) (end 111.76 111.76) (width 5) (layer F.Cu) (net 17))
 (segment (start 111.76 111.76) (end 111.76 110.49) (width 5) (layer F.Cu) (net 17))
 (segment (start 113.03 109.22) (end 111.76 111.76) (width 5) (layer F.Cu) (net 17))
 (segment (start 160.02 118.745) (end 160.02 109.22) (width 5) (layer F.Cu) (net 17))
 (segment (start 201.83 109.22) (end 160.02 109.22) (width 5) (layer F.Cu) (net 17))
 (segment (start 208.28 112.495) (end 205.005 109.22) (width 5) (layer F.Cu) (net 17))
 (segment (start 205.005 109.22) (end 201.83 109.22) (width 5) (layer F.Cu) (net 17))
 (segment (start 208.28 118.745) (end 208.28 112.495) (width 5) (layer F.Cu) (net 17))
 (segment (start 68.23 59.46) (end 73.43 59.46) (width 5) (layer F.Cu) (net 32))
 (segment (start 119.527766 59.46) (end 119.551766 59.436) (width 5) (layer F.Cu) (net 28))
 (segment (start 117.76 59.46) (end 119.527766 59.46) (width 5) (layer F.Cu) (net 28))
 (segment (start 119.551766 59.436) (end 122.682 59.436) (width 5) (layer F.Cu) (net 28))
 (segment (start 166.02 59.46) (end 170.434 59.46) (width 5) (layer F.Cu) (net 25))
 (segment (start 216.047766 59.46) (end 216.071766 59.436) (width 5) (layer F.Cu) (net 30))
 (segment (start 214.28 59.46) (end 216.047766 59.46) (width 5) (layer F.Cu) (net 30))
 (segment (start 214.28 59.46) (end 219.686 59.46) (width 5) (layer F.Cu) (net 30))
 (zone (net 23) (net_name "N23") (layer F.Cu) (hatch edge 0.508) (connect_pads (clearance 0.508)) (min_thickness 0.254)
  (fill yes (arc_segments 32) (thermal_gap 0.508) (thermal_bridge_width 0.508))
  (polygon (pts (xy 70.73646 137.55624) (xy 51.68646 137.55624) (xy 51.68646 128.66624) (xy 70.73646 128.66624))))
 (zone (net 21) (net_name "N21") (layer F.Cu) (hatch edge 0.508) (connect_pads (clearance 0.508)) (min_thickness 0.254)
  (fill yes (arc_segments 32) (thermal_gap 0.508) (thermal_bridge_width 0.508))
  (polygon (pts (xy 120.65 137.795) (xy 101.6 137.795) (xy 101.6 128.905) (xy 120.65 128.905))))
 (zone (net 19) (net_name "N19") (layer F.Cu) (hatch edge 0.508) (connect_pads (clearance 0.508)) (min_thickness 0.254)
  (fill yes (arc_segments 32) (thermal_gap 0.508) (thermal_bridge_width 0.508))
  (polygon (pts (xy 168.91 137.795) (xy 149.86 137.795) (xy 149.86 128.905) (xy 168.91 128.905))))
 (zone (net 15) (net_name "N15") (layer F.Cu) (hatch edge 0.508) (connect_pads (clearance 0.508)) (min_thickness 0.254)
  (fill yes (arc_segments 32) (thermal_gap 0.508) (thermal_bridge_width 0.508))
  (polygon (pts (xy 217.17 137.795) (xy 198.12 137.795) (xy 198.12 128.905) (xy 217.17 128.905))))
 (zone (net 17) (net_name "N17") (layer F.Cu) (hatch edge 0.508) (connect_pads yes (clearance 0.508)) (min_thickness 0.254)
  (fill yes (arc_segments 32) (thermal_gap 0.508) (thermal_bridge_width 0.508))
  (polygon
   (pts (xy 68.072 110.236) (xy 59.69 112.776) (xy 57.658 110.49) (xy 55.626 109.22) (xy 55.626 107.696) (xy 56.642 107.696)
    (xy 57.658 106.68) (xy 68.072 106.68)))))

